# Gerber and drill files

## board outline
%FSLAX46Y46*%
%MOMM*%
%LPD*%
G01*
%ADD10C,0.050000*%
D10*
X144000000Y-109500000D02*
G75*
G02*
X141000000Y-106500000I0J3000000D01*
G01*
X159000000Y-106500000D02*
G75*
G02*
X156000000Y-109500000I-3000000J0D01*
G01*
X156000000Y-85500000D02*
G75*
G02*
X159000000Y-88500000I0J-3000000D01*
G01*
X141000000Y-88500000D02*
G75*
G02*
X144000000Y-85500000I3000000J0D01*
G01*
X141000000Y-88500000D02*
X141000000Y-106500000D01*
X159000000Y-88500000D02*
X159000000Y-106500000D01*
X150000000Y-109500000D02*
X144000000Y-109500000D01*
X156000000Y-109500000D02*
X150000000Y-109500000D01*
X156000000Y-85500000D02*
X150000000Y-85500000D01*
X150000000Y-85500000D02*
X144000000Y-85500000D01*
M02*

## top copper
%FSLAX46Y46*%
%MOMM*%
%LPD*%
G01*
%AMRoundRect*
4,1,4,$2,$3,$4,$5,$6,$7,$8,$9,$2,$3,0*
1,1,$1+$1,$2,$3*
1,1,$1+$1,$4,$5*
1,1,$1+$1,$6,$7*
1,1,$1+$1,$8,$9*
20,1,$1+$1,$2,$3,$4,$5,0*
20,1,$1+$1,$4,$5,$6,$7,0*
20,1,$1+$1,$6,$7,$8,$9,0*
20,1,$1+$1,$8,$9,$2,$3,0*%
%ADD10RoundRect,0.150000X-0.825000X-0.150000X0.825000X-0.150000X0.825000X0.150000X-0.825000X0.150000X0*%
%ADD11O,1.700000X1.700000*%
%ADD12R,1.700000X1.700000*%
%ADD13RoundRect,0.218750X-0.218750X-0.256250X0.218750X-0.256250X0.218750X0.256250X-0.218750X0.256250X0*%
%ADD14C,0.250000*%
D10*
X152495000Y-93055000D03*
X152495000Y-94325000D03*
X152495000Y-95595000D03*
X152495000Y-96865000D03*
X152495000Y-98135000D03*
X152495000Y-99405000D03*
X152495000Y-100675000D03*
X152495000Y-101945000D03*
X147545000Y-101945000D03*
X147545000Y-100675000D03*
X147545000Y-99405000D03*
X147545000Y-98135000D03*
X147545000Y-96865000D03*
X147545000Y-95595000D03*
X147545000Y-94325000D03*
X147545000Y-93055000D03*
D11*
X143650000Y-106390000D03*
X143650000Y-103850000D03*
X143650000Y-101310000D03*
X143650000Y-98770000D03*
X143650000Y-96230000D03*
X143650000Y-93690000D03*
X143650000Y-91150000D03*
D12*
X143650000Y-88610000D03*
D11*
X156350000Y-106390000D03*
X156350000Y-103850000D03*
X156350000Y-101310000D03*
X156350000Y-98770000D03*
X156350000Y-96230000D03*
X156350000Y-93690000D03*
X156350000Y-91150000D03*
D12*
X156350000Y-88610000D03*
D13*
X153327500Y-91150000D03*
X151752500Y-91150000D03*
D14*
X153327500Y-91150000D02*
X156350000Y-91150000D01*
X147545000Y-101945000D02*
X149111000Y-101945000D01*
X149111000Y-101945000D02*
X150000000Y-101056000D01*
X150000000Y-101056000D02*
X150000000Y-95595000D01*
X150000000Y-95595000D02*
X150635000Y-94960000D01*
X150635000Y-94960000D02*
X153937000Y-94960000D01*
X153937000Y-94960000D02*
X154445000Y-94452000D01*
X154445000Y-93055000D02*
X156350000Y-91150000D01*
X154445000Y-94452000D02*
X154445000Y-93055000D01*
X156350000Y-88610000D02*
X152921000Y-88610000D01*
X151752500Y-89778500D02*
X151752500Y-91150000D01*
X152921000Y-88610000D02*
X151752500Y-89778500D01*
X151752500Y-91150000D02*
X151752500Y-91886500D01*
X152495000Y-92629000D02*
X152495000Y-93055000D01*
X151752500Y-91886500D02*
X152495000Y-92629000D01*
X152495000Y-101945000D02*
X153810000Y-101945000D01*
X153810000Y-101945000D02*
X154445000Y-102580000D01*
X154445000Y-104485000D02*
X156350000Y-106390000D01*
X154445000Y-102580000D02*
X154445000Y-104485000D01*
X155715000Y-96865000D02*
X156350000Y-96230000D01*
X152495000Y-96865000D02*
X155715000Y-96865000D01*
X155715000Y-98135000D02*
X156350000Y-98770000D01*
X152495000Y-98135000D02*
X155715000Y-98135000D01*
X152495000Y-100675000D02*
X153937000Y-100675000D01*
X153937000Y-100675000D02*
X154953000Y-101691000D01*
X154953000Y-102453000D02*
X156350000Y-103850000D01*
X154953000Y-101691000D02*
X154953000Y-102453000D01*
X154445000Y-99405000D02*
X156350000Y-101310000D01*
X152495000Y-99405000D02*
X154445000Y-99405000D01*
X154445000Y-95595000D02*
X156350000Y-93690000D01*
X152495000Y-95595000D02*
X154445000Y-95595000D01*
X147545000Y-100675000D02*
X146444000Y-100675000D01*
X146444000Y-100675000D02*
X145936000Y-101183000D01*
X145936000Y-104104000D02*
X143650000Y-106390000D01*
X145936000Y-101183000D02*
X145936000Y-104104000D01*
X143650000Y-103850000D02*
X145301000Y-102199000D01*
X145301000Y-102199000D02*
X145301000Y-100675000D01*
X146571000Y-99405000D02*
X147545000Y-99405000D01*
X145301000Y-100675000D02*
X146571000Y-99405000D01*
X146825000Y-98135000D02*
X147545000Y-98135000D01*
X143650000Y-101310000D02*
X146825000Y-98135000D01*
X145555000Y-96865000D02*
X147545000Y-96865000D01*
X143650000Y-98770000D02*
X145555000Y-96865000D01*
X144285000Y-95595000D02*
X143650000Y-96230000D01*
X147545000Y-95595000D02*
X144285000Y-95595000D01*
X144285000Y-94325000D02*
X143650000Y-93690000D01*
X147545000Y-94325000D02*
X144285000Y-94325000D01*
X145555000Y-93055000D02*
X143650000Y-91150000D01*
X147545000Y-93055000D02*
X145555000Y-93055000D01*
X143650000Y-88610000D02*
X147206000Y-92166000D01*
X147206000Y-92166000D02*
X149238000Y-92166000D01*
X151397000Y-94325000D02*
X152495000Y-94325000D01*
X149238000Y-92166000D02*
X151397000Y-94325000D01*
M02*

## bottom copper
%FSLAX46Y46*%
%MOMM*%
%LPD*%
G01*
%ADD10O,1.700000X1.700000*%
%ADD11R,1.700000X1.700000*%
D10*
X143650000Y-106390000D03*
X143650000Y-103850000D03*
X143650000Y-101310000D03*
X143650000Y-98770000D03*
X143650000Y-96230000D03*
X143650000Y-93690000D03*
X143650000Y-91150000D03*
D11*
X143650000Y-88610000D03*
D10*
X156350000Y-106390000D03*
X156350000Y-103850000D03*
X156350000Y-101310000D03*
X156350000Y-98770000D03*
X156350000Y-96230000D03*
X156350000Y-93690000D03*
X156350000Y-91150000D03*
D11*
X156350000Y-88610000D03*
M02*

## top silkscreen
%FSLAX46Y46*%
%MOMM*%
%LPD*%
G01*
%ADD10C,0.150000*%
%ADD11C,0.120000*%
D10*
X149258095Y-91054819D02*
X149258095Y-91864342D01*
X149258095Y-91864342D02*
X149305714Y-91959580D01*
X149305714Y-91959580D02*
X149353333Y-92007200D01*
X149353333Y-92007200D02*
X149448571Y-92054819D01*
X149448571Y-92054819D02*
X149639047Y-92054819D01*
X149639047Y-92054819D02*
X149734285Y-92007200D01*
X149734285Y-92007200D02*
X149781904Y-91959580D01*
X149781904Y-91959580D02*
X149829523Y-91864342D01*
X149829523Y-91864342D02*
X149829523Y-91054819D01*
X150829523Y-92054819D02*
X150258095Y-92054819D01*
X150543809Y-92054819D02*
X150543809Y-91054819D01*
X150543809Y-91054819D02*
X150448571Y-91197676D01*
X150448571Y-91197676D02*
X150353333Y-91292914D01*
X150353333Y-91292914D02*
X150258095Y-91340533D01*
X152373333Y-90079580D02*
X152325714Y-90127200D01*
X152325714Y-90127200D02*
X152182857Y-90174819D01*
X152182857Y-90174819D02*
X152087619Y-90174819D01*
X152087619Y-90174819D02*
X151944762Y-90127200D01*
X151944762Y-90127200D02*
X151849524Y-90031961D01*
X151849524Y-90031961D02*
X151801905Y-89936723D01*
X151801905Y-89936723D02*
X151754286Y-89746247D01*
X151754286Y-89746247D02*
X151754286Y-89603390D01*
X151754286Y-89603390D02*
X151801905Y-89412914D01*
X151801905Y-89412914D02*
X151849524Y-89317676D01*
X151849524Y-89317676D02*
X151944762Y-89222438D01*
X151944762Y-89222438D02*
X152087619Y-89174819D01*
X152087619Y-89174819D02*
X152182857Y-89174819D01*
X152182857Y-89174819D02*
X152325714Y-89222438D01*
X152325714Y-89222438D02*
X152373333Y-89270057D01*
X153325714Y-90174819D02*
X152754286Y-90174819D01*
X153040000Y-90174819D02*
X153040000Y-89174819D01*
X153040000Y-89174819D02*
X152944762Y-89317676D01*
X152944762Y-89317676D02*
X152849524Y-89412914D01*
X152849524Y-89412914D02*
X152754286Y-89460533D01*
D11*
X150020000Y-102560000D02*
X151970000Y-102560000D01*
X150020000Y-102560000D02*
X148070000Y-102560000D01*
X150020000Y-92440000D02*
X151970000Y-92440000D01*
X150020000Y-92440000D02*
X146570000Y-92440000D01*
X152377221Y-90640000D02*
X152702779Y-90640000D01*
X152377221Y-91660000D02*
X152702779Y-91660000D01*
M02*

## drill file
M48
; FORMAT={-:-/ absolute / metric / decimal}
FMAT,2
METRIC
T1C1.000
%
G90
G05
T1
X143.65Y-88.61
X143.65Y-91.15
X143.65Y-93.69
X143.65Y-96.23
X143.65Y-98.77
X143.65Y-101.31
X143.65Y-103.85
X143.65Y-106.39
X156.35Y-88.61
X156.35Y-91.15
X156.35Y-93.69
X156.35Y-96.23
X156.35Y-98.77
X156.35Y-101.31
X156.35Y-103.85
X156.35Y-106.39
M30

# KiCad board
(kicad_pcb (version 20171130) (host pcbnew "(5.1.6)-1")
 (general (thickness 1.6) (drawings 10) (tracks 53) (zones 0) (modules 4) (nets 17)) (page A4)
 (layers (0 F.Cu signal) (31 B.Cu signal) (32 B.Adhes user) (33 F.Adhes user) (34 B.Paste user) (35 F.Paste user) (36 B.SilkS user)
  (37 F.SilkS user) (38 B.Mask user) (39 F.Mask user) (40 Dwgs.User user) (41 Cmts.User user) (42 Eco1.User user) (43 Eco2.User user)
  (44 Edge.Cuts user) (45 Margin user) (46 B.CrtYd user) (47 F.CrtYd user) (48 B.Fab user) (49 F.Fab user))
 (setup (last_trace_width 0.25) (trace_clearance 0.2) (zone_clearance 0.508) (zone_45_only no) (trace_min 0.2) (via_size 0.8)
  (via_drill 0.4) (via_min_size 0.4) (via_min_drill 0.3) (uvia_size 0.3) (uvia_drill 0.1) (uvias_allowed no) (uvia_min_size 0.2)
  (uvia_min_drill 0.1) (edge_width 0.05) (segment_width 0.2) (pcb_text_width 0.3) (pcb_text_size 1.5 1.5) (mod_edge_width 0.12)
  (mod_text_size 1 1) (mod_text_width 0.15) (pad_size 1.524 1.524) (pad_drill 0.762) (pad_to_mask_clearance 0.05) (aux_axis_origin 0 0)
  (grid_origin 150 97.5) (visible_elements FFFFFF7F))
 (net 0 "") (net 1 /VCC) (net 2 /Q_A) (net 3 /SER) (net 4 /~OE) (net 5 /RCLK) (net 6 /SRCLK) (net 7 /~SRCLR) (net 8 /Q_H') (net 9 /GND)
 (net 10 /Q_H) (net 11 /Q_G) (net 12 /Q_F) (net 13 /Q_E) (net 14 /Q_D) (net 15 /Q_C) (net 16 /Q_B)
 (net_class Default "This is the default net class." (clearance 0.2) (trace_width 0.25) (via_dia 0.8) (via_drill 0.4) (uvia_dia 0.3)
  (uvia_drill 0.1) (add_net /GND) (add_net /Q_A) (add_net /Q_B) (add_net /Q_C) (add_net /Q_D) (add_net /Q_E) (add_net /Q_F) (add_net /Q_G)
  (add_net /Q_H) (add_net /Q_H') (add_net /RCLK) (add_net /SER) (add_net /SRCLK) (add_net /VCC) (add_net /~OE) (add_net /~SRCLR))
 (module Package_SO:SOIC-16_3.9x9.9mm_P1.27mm (layer F.Cu) (at 150.02 97.5)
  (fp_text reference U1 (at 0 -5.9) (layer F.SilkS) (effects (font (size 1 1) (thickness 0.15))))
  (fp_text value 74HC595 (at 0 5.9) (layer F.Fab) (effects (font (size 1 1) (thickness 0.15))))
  (fp_line (start 0 5.06) (end 1.95 5.06) (layer F.SilkS) (width 0.12))
  (fp_line (start 0 5.06) (end -1.95 5.06) (layer F.SilkS) (width 0.12))
  (fp_line (start 0 -5.06) (end 1.95 -5.06) (layer F.SilkS) (width 0.12))
  (fp_line (start 0 -5.06) (end -3.45 -5.06) (layer F.SilkS) (width 0.12))
  (pad 16 smd roundrect (at 2.475 -4.445) (size 1.95 0.6) (layers F.Cu F.Paste F.Mask) (roundrect_rratio 0.25) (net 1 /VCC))
  (pad 15 smd roundrect (at 2.475 -3.175) (size 1.95 0.6) (layers F.Cu F.Paste F.Mask) (roundrect_rratio 0.25) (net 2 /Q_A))
  (pad 14 smd roundrect (at 2.475 -1.905) (size 1.95 0.6) (layers F.Cu F.Paste F.Mask) (roundrect_rratio 0.25) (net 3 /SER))
  (pad 13 smd roundrect (at 2.475 -0.635) (size 1.95 0.6) (layers F.Cu F.Paste F.Mask) (roundrect_rratio 0.25) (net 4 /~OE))
  (pad 12 smd roundrect (at 2.475 0.635) (size 1.95 0.6) (layers F.Cu F.Paste F.Mask) (roundrect_rratio 0.25) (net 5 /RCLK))
  (pad 11 smd roundrect (at 2.475 1.905) (size 1.95 0.6) (layers F.Cu F.Paste F.Mask) (roundrect_rratio 0.25) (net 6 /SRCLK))
  (pad 10 smd roundrect (at 2.475 3.175) (size 1.95 0.6) (layers F.Cu F.Paste F.Mask) (roundrect_rratio 0.25) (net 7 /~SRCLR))
  (pad 9 smd roundrect (at 2.475 4.445) (size 1.95 0.6) (layers F.Cu F.Paste F.Mask) (roundrect_rratio 0.25) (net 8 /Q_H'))
  (pad 8 smd roundrect (at -2.475 4.445) (size 1.95 0.6) (layers F.Cu F.Paste F.Mask) (roundrect_rratio 0.25) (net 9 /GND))
  (pad 7 smd roundrect (at -2.475 3.175) (size 1.95 0.6) (layers F.Cu F.Paste F.Mask) (roundrect_rratio 0.25) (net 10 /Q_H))
  (pad 6 smd roundrect (at -2.475 1.905) (size 1.95 0.6) (layers F.Cu F.Paste F.Mask) (roundrect_rratio 0.25) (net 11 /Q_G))
  (pad 5 smd roundrect (at -2.475 0.635) (size 1.95 0.6) (layers F.Cu F.Paste F.Mask) (roundrect_rratio 0.25) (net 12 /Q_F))
  (pad 4 smd roundrect (at -2.475 -0.635) (size 1.95 0.6) (layers F.Cu F.Paste F.Mask) (roundrect_rratio 0.25) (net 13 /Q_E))
  (pad 3 smd roundrect (at -2.475 -1.905) (size 1.95 0.6) (layers F.Cu F.Paste F.Mask) (roundrect_rratio 0.25) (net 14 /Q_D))
  (pad 2 smd roundrect (at -2.475 -3.175) (size 1.95 0.6) (layers F.Cu F.Paste F.Mask) (roundrect_rratio 0.25) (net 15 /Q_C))
  (pad 1 smd roundrect (at -2.475 -4.445) (size 1.95 0.6) (layers F.Cu F.Paste F.Mask) (roundrect_rratio 0.25) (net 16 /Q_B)))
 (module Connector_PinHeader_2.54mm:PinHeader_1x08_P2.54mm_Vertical (layer B.Cu) (at 143.65 88.61 180)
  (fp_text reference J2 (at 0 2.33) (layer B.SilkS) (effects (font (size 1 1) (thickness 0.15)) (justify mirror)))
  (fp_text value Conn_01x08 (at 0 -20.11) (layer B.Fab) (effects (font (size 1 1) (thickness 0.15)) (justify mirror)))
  (pad 8 thru_hole oval (at 0 -17.78 180) (size 1.7 1.7) (drill 1) (layers *.Cu *.Mask) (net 10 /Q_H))
  (pad 7 thru_hole oval (at 0 -15.24 180) (size 1.7 1.7) (drill 1) (layers *.Cu *.Mask) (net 11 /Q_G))
  (pad 6 thru_hole oval (at 0 -12.7 180) (size 1.7 1.7) (drill 1) (layers *.Cu *.Mask) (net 12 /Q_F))
  (pad 5 thru_hole oval (at 0 -10.16 180) (size 1.7 1.7) (drill 1) (layers *.Cu *.Mask) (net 13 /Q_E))
  (pad 4 thru_hole oval (at 0 -7.62 180) (size 1.7 1.7) (drill 1) (layers *.Cu *.Mask) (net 14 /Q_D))
  (pad 3 thru_hole oval (at 0 -5.08 180) (size 1.7 1.7) (drill 1) (layers *.Cu *.Mask) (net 15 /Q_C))
  (pad 2 thru_hole oval (at 0 -2.54 180) (size 1.7 1.7) (drill 1) (layers *.Cu *.Mask) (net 16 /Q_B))
  (pad 1 thru_hole rect (at 0 0 180) (size 1.7 1.7) (drill 1) (layers *.Cu *.Mask) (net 2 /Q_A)))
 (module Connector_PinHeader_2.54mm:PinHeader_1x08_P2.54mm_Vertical (layer B.Cu) (at 156.35 88.61 180)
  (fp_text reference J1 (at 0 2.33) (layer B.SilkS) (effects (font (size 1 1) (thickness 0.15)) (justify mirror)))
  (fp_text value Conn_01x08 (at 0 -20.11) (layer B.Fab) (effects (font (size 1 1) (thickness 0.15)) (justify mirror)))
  (pad 8 thru_hole oval (at 0 -17.78 180) (size 1.7 1.7) (drill 1) (layers *.Cu *.Mask) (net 8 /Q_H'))
  (pad 7 thru_hole oval (at 0 -15.24 180) (size 1.7 1.7) (drill 1) (layers *.Cu *.Mask) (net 7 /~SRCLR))
  (pad 6 thru_hole oval (at 0 -12.7 180) (size 1.7 1.7) (drill 1) (layers *.Cu *.Mask) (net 6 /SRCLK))
  (pad 5 thru_hole oval (at 0 -10.16 180) (size 1.7 1.7) (drill 1) (layers *.Cu *.Mask) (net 5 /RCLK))
  (pad 4 thru_hole oval (at 0 -7.62 180) (size 1.7 1.7) (drill 1) (layers *.Cu *.Mask) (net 4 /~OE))
  (pad 3 thru_hole oval (at 0 -5.08 180) (size 1.7 1.7) (drill 1) (layers *.Cu *.Mask) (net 3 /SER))
  (pad 2 thru_hole oval (at 0 -2.54 180) (size 1.7 1.7) (drill 1) (layers *.Cu *.Mask) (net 9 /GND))
  (pad 1 thru_hole rect (at 0 0 180) (size 1.7 1.7) (drill 1) (layers *.Cu *.Mask) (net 1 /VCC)))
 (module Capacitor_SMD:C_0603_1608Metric (layer F.Cu) (at 152.54 91.15)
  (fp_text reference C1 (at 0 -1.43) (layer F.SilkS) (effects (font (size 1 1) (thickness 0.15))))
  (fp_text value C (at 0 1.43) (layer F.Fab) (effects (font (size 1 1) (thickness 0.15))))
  (fp_line (start -0.162779 -0.51) (end 0.162779 -0.51) (layer F.SilkS) (width 0.12))
  (fp_line (start -0.162779 0.51) (end 0.162779 0.51) (layer F.SilkS) (width 0.12))
  (pad 2 smd roundrect (at 0.7875 0) (size 0.875 0.95) (layers F.Cu F.Paste F.Mask) (roundrect_rratio 0.25) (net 9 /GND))
  (pad 1 smd roundrect (at -0.7875 0) (size 0.875 0.95) (layers F.Cu F.Paste F.Mask) (roundrect_rratio 0.25) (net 1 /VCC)))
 (gr_arc (start 144 106.5) (end 141 106.5) (angle -90) (layer Edge.Cuts) (width 0.05))
 (gr_arc (start 156 106.5) (end 156 109.5) (angle -90) (layer Edge.Cuts) (width 0.05))
 (gr_arc (start 156 88.5) (end 159 88.5) (angle -90) (layer Edge.Cuts) (width 0.05))
 (gr_arc (start 144 88.5) (end 144 85.5) (angle -90) (layer Edge.Cuts) (width 0.05))
 (gr_line (start 141 88.5) (end 141 106.5) (layer Edge.Cuts) (width 0.05))
 (gr_line (start 159 88.5) (end 159 106.5) (layer Edge.Cuts) (width 0.05))
 (gr_line (start 150 109.5) (end 144 109.5) (layer Edge.Cuts) (width 0.05))
 (gr_line (start 156 109.5) (end 150 109.5) (layer Edge.Cuts) (width 0.05))
 (gr_line (start 156 85.5) (end 150 85.5) (layer Edge.Cuts) (width 0.05))
 (gr_line (start 150 85.5) (end 144 85.5) (layer Edge.Cuts) (width 0.05))
 (segment (start 153.3275 91.15) (end 156.35 91.15) (width 0.25) (layer F.Cu) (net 9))
 (segment (start 147.545 101.945) (end 149.111 101.945) (width 0.25) (layer F.Cu) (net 9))
 (segment (start 149.111 101.945) (end 150 101.056) (width 0.25) (layer F.Cu) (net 9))
 (segment (start 150 101.056) (end 150 95.595) (width 0.25) (layer F.Cu) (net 9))
 (segment (start 150 95.595) (end 150.635 94.96) (width 0.25) (layer F.Cu) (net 9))
 (segment (start 150.635 94.96) (end 153.937 94.96) (width 0.25) (layer F.Cu) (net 9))
 (segment (start 153.937 94.96) (end 154.445 94.452) (width 0.25) (layer F.Cu) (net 9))
 (segment (start 154.445 93.055) (end 156.35 91.15) (width 0.25) (layer F.Cu) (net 9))
 (segment (start 154.445 94.452) (end 154.445 93.055) (width 0.25) (layer F.Cu) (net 9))
 (segment (start 156.35 88.61) (end 152.921 88.61) (width 0.25) (layer F.Cu) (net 1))
 (segment (start 151.7525 89.7785) (end 151.7525 91.15) (width 0.25) (layer F.Cu) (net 1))
 (segment (start 152.921 88.61) (end 151.7525 89.7785) (width 0.25) (layer F.Cu) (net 1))
 (segment (start 151.7525 91.15) (end 151.7525 91.8865) (width 0.25) (layer F.Cu) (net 1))
 (segment (start 152.495 92.629) (end 152.495 93.055) (width 0.25) (layer F.Cu) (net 1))
 (segment (start 151.7525 91.8865) (end 152.495 92.629) (width 0.25) (layer F.Cu) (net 1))
 (segment (start 152.495 101.945) (end 153.81 101.945) (width 0.25) (layer F.Cu) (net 8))
 (segment (start 153.81 101.945) (end 154.445 102.58) (width 0.25) (layer F.Cu) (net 8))
 (segment (start 154.445 104.485) (end 156.35 106.39) (width 0.25) (layer F.Cu) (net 8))
 (segment (start 154.445 102.58) (end 154.445 104.485) (width 0.25) (layer F.Cu) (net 8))
 (segment (start 155.715 96.865) (end 156.35 96.23) (width 0.25) (layer F.Cu) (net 4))
 (segment (start 152.495 96.865) (end 155.715 96.865) (width 0.25) (layer F.Cu) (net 4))
 (segment (start 155.715 98.135) (end 156.35 98.77) (width 0.25) (layer F.Cu) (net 5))
 (segment (start 152.495 98.135) (end 155.715 98.135) (width 0.25) (layer F.Cu) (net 5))
 (segment (start 152.495 100.675) (end 153.937 100.675) (width 0.25) (layer F.Cu) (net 7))
 (segment (start 153.937 100.675) (end 154.953 101.691) (width 0.25) (layer F.Cu) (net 7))
 (segment (start 154.953 102.453) (end 156.35 103.85) (width 0.25) (layer F.Cu) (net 7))
 (segment (start 154.953 101.691) (end 154.953 102.453) (width 0.25) (layer F.Cu) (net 7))
 (segment (start 154.445 99.405) (end 156.35 101.31) (width 0.25) (layer F.Cu) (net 6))
 (segment (start 152.495 99.405) (end 154.445 99.405) (width 0.25) (layer F.Cu) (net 6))
 (segment (start 154.445 95.595) (end 156.35 93.69) (width 0.25) (layer F.Cu) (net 3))
 (segment (start 152.495 95.595) (end 154.445 95.595) (width 0.25) (layer F.Cu) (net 3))
 (segment (start 147.545 100.675) (end 146.444 100.675) (width 0.25) (layer F.Cu) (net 10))
 (segment (start 146.444 100.675) (end 145.936 101.183) (width 0.25) (layer F.Cu) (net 10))
 (segment (start 145.936 104.104) (end 143.65 106.39) (width 0.25) (layer F.Cu) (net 10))
 (segment (start 145.936 101.183) (end 145.936 104.104) (width 0.25) (layer F.Cu) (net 10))
 (segment (start 143.65 103.85) (end 145.301 102.199) (width 0.25) (layer F.Cu) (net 11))
 (segment (start 145.301 102.199) (end 145.301 100.675) (width 0.25) (layer F.Cu) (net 11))
 (segment (start 146.571 99.405) (end 147.545 99.405) (width 0.25) (layer F.Cu) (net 11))
 (segment (start 145.301 100.675) (end 146.571 99.405) (width 0.25) (layer F.Cu) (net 11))
 (segment (start 146.825 98.135) (end 147.545 98.135) (width 0.25) (layer F.Cu) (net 12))
 (segment (start 143.65 101.31) (end 146.825 98.135) (width 0.25) (layer F.Cu) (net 12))
 (segment (start 145.555 96.865) (end 147.545 96.865) (width 0.25) (layer F.Cu) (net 13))
 (segment (start 143.65 98.77) (end 145.555 96.865) (width 0.25) (layer F.Cu) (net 13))
 (segment (start 144.285 95.595) (end 143.65 96.23) (width 0.25) (layer F.Cu) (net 14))
 (segment (start 147.545 95.595) (end 144.285 95.595) (width 0.25) (layer F.Cu) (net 14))
 (segment (start 144.285 94.325) (end 143.65 93.69) (width 0.25) (layer F.Cu) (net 15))
 (segment (start 147.545 94.325) (end 144.285 94.325) (width 0.25) (layer F.Cu) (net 15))
 (segment (start 145.555 93.055) (end 143.65 91.15) (width 0.25) (layer F.Cu) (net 16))
 (segment (start 147.545 93.055) (end 145.555 93.055) (width 0.25) (layer F.Cu) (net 16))
 (segment (start 143.65 88.61) (end 147.206 92.166) (width 0.25) (layer F.Cu) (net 2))
 (segment (start 147.206 92.166) (end 149.238 92.166) (width 0.25) (layer F.Cu) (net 2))
 (segment (start 151.397 94.325) (end 152.495 94.325) (width 0.25) (layer F.Cu) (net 2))
 (segment (start 149.238 92.166) (end 151.397 94.325) (width 0.25) (layer F.Cu) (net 2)))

